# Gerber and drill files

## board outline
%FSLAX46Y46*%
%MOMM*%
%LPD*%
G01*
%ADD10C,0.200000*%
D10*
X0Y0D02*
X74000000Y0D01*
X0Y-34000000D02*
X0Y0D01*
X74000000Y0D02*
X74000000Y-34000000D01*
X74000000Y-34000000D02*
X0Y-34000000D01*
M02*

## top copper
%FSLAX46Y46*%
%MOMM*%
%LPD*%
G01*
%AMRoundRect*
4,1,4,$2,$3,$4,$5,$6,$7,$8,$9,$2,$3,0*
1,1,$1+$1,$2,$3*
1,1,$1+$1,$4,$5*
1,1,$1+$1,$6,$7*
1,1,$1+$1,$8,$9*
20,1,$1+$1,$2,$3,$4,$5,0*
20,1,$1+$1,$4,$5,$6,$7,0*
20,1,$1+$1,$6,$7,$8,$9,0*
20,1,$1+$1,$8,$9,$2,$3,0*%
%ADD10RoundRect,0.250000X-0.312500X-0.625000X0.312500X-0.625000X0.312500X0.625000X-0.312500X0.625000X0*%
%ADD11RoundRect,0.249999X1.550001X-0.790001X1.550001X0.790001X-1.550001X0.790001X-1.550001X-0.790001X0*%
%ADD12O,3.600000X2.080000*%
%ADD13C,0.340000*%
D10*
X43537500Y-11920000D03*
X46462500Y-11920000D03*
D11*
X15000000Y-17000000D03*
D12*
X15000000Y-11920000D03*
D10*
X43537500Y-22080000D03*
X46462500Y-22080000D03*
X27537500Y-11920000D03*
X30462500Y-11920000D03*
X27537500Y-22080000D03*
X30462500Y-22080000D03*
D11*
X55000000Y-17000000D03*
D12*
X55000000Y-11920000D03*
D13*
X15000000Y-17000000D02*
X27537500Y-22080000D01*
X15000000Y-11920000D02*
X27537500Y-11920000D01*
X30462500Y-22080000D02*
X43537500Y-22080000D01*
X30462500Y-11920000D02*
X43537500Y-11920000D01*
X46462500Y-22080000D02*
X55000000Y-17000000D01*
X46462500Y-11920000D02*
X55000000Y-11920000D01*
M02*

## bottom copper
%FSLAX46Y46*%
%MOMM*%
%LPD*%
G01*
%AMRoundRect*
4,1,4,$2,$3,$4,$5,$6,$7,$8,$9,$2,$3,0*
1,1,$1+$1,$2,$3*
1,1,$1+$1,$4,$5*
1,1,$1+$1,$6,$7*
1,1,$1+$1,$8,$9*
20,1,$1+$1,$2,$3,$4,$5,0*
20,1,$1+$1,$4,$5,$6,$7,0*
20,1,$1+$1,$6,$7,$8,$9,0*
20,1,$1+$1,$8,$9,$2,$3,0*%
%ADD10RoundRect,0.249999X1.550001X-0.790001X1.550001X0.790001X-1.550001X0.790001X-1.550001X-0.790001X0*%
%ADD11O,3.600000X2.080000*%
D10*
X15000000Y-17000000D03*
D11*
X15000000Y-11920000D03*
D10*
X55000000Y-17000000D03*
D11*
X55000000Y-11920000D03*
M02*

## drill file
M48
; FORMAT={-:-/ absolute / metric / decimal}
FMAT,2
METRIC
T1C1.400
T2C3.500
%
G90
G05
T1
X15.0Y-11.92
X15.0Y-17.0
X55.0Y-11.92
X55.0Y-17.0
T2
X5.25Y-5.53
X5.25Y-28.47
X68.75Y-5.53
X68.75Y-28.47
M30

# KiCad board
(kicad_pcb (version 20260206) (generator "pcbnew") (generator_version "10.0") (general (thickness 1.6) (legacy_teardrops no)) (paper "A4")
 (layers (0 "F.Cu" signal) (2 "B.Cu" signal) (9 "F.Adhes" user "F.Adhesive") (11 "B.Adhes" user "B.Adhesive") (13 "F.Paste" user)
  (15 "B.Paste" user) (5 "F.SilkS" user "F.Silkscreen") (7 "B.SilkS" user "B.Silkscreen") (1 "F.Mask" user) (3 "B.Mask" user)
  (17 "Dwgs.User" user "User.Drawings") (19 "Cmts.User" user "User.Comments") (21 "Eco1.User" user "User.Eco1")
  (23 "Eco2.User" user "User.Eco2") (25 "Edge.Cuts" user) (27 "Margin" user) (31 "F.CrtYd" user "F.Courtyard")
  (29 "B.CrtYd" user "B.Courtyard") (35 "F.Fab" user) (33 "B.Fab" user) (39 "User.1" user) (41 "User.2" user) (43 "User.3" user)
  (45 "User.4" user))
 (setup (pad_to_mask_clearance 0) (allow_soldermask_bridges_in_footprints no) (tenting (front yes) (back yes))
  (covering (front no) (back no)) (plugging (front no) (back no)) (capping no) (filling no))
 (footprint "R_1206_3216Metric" (layer "F.Cu") (at 45 11.92)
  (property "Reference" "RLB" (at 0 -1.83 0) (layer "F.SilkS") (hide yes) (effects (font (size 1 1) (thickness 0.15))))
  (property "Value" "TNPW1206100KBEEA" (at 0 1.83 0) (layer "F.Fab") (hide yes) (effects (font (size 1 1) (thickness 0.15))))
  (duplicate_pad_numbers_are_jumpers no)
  (pad "1" smd roundrect (at -1.4625 0) (size 1.125 1.75) (layers "F.Cu" "F.Mask" "F.Paste") (roundrect_rratio 0.222222) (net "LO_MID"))
  (pad "2" smd roundrect (at 1.4625 0) (size 1.125 1.75) (layers "F.Cu" "F.Mask" "F.Paste") (roundrect_rratio 0.222222) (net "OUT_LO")))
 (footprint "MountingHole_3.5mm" (layer "F.Cu") (at 5.25 5.53)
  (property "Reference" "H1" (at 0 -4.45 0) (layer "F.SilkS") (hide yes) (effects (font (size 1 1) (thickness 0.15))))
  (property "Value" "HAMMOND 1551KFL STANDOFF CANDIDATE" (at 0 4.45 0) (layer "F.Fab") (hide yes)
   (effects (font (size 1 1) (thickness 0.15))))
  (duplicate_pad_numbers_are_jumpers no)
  (pad "" np_thru_hole circle (at 0 0) (size 3.5 3.5) (drill 3.5) (layers "*.Cu" "*.Mask")))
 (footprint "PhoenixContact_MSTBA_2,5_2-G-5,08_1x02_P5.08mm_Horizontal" (layer "F.Cu") (at 15 17 90)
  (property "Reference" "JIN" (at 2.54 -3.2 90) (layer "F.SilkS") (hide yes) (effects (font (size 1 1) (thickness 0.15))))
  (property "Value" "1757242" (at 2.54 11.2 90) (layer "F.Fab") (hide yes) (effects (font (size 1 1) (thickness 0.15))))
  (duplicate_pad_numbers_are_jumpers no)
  (pad "1" thru_hole roundrect (at 0 0 90) (size 2.08 3.6) (drill 1.4) (layers "*.Cu" "*.Mask") (remove_unused_layers no)
   (roundrect_rratio 0.120192) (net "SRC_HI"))
  (pad "2" thru_hole oval (at 5.08 0 90) (size 2.08 3.6) (drill 1.4) (layers "*.Cu" "*.Mask") (remove_unused_layers no) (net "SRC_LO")))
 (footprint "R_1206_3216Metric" (layer "F.Cu") (at 45 22.08)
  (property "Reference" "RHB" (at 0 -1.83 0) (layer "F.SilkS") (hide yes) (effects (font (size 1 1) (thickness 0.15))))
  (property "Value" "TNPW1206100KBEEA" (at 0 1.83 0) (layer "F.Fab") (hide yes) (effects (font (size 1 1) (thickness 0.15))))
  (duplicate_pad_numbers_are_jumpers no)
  (pad "1" smd roundrect (at -1.4625 0) (size 1.125 1.75) (layers "F.Cu" "F.Mask" "F.Paste") (roundrect_rratio 0.222222) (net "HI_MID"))
  (pad "2" smd roundrect (at 1.4625 0) (size 1.125 1.75) (layers "F.Cu" "F.Mask" "F.Paste") (roundrect_rratio 0.222222) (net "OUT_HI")))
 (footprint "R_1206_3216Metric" (layer "F.Cu") (at 29 11.92)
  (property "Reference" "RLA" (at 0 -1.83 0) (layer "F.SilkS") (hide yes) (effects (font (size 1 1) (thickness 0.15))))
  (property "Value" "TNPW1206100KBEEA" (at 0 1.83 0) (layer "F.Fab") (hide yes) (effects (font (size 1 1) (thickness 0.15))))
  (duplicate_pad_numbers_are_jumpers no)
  (pad "1" smd roundrect (at -1.4625 0) (size 1.125 1.75) (layers "F.Cu" "F.Mask" "F.Paste") (roundrect_rratio 0.222222) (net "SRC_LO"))
  (pad "2" smd roundrect (at 1.4625 0) (size 1.125 1.75) (layers "F.Cu" "F.Mask" "F.Paste") (roundrect_rratio 0.222222) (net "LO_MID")))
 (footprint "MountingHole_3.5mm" (layer "F.Cu") (at 5.25 28.47)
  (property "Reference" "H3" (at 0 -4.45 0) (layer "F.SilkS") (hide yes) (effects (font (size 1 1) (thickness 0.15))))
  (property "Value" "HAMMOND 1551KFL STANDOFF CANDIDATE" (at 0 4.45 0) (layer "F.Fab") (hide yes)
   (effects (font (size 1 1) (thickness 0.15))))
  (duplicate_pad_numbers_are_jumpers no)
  (pad "" np_thru_hole circle (at 0 0) (size 3.5 3.5) (drill 3.5) (layers "*.Cu" "*.Mask")))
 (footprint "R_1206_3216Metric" (layer "F.Cu") (at 29 22.08)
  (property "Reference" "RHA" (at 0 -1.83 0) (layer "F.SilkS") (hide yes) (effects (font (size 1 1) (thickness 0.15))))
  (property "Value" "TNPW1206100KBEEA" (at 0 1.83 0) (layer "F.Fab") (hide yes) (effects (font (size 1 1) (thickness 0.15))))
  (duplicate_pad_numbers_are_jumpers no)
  (pad "1" smd roundrect (at -1.4625 0) (size 1.125 1.75) (layers "F.Cu" "F.Mask" "F.Paste") (roundrect_rratio 0.222222) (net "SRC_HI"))
  (pad "2" smd roundrect (at 1.4625 0) (size 1.125 1.75) (layers "F.Cu" "F.Mask" "F.Paste") (roundrect_rratio 0.222222) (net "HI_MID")))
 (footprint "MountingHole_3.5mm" (layer "F.Cu") (at 68.75 28.47)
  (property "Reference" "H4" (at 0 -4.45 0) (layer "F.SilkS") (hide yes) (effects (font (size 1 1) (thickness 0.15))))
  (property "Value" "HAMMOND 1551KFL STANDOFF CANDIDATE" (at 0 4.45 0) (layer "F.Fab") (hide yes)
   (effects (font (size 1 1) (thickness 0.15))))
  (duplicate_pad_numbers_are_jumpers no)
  (pad "" np_thru_hole circle (at 0 0) (size 3.5 3.5) (drill 3.5) (layers "*.Cu" "*.Mask")))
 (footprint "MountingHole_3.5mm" (layer "F.Cu") (at 68.75 5.53)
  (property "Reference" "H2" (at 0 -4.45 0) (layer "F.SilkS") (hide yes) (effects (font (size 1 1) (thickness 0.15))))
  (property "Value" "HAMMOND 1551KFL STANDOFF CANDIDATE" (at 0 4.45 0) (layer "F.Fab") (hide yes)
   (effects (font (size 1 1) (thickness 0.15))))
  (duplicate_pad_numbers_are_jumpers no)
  (pad "" np_thru_hole circle (at 0 0) (size 3.5 3.5) (drill 3.5) (layers "*.Cu" "*.Mask")))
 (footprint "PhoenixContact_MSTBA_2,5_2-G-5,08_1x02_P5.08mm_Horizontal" (layer "F.Cu") (at 55 17 90)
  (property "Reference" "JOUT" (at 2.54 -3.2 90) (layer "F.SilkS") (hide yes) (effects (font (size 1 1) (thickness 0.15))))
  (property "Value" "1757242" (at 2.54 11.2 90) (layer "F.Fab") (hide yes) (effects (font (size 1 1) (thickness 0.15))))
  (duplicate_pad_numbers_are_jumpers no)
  (pad "1" thru_hole roundrect (at 0 0 90) (size 2.08 3.6) (drill 1.4) (layers "*.Cu" "*.Mask") (remove_unused_layers no)
   (roundrect_rratio 0.120192) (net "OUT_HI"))
  (pad "2" thru_hole oval (at 5.08 0 90) (size 2.08 3.6) (drill 1.4) (layers "*.Cu" "*.Mask") (remove_unused_layers no) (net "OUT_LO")))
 (gr_line (start 0 0) (end 74 0) (stroke (width 0.2) (type default)) (layer "Edge.Cuts"))
 (gr_line (start 0 34) (end 0 0) (stroke (width 0.2) (type default)) (layer "Edge.Cuts"))
 (gr_line (start 74 0) (end 74 34) (stroke (width 0.2) (type default)) (layer "Edge.Cuts"))
 (gr_line (start 74 34) (end 0 34) (stroke (width 0.2) (type default)) (layer "Edge.Cuts"))
 (segment (start 15 17) (end 27.5375 22.08) (width 0.34) (layer "F.Cu") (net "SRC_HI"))
 (segment (start 15 11.92) (end 27.5375 11.92) (width 0.34) (layer "F.Cu") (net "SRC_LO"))
 (segment (start 30.4625 22.08) (end 43.5375 22.08) (width 0.34) (layer "F.Cu") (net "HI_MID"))
 (segment (start 30.4625 11.92) (end 43.5375 11.92) (width 0.34) (layer "F.Cu") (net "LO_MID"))
 (segment (start 46.4625 22.08) (end 55 17) (width 0.34) (layer "F.Cu") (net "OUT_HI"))
 (segment (start 46.4625 11.92) (end 55 11.92) (width 0.34) (layer "F.Cu") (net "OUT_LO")))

